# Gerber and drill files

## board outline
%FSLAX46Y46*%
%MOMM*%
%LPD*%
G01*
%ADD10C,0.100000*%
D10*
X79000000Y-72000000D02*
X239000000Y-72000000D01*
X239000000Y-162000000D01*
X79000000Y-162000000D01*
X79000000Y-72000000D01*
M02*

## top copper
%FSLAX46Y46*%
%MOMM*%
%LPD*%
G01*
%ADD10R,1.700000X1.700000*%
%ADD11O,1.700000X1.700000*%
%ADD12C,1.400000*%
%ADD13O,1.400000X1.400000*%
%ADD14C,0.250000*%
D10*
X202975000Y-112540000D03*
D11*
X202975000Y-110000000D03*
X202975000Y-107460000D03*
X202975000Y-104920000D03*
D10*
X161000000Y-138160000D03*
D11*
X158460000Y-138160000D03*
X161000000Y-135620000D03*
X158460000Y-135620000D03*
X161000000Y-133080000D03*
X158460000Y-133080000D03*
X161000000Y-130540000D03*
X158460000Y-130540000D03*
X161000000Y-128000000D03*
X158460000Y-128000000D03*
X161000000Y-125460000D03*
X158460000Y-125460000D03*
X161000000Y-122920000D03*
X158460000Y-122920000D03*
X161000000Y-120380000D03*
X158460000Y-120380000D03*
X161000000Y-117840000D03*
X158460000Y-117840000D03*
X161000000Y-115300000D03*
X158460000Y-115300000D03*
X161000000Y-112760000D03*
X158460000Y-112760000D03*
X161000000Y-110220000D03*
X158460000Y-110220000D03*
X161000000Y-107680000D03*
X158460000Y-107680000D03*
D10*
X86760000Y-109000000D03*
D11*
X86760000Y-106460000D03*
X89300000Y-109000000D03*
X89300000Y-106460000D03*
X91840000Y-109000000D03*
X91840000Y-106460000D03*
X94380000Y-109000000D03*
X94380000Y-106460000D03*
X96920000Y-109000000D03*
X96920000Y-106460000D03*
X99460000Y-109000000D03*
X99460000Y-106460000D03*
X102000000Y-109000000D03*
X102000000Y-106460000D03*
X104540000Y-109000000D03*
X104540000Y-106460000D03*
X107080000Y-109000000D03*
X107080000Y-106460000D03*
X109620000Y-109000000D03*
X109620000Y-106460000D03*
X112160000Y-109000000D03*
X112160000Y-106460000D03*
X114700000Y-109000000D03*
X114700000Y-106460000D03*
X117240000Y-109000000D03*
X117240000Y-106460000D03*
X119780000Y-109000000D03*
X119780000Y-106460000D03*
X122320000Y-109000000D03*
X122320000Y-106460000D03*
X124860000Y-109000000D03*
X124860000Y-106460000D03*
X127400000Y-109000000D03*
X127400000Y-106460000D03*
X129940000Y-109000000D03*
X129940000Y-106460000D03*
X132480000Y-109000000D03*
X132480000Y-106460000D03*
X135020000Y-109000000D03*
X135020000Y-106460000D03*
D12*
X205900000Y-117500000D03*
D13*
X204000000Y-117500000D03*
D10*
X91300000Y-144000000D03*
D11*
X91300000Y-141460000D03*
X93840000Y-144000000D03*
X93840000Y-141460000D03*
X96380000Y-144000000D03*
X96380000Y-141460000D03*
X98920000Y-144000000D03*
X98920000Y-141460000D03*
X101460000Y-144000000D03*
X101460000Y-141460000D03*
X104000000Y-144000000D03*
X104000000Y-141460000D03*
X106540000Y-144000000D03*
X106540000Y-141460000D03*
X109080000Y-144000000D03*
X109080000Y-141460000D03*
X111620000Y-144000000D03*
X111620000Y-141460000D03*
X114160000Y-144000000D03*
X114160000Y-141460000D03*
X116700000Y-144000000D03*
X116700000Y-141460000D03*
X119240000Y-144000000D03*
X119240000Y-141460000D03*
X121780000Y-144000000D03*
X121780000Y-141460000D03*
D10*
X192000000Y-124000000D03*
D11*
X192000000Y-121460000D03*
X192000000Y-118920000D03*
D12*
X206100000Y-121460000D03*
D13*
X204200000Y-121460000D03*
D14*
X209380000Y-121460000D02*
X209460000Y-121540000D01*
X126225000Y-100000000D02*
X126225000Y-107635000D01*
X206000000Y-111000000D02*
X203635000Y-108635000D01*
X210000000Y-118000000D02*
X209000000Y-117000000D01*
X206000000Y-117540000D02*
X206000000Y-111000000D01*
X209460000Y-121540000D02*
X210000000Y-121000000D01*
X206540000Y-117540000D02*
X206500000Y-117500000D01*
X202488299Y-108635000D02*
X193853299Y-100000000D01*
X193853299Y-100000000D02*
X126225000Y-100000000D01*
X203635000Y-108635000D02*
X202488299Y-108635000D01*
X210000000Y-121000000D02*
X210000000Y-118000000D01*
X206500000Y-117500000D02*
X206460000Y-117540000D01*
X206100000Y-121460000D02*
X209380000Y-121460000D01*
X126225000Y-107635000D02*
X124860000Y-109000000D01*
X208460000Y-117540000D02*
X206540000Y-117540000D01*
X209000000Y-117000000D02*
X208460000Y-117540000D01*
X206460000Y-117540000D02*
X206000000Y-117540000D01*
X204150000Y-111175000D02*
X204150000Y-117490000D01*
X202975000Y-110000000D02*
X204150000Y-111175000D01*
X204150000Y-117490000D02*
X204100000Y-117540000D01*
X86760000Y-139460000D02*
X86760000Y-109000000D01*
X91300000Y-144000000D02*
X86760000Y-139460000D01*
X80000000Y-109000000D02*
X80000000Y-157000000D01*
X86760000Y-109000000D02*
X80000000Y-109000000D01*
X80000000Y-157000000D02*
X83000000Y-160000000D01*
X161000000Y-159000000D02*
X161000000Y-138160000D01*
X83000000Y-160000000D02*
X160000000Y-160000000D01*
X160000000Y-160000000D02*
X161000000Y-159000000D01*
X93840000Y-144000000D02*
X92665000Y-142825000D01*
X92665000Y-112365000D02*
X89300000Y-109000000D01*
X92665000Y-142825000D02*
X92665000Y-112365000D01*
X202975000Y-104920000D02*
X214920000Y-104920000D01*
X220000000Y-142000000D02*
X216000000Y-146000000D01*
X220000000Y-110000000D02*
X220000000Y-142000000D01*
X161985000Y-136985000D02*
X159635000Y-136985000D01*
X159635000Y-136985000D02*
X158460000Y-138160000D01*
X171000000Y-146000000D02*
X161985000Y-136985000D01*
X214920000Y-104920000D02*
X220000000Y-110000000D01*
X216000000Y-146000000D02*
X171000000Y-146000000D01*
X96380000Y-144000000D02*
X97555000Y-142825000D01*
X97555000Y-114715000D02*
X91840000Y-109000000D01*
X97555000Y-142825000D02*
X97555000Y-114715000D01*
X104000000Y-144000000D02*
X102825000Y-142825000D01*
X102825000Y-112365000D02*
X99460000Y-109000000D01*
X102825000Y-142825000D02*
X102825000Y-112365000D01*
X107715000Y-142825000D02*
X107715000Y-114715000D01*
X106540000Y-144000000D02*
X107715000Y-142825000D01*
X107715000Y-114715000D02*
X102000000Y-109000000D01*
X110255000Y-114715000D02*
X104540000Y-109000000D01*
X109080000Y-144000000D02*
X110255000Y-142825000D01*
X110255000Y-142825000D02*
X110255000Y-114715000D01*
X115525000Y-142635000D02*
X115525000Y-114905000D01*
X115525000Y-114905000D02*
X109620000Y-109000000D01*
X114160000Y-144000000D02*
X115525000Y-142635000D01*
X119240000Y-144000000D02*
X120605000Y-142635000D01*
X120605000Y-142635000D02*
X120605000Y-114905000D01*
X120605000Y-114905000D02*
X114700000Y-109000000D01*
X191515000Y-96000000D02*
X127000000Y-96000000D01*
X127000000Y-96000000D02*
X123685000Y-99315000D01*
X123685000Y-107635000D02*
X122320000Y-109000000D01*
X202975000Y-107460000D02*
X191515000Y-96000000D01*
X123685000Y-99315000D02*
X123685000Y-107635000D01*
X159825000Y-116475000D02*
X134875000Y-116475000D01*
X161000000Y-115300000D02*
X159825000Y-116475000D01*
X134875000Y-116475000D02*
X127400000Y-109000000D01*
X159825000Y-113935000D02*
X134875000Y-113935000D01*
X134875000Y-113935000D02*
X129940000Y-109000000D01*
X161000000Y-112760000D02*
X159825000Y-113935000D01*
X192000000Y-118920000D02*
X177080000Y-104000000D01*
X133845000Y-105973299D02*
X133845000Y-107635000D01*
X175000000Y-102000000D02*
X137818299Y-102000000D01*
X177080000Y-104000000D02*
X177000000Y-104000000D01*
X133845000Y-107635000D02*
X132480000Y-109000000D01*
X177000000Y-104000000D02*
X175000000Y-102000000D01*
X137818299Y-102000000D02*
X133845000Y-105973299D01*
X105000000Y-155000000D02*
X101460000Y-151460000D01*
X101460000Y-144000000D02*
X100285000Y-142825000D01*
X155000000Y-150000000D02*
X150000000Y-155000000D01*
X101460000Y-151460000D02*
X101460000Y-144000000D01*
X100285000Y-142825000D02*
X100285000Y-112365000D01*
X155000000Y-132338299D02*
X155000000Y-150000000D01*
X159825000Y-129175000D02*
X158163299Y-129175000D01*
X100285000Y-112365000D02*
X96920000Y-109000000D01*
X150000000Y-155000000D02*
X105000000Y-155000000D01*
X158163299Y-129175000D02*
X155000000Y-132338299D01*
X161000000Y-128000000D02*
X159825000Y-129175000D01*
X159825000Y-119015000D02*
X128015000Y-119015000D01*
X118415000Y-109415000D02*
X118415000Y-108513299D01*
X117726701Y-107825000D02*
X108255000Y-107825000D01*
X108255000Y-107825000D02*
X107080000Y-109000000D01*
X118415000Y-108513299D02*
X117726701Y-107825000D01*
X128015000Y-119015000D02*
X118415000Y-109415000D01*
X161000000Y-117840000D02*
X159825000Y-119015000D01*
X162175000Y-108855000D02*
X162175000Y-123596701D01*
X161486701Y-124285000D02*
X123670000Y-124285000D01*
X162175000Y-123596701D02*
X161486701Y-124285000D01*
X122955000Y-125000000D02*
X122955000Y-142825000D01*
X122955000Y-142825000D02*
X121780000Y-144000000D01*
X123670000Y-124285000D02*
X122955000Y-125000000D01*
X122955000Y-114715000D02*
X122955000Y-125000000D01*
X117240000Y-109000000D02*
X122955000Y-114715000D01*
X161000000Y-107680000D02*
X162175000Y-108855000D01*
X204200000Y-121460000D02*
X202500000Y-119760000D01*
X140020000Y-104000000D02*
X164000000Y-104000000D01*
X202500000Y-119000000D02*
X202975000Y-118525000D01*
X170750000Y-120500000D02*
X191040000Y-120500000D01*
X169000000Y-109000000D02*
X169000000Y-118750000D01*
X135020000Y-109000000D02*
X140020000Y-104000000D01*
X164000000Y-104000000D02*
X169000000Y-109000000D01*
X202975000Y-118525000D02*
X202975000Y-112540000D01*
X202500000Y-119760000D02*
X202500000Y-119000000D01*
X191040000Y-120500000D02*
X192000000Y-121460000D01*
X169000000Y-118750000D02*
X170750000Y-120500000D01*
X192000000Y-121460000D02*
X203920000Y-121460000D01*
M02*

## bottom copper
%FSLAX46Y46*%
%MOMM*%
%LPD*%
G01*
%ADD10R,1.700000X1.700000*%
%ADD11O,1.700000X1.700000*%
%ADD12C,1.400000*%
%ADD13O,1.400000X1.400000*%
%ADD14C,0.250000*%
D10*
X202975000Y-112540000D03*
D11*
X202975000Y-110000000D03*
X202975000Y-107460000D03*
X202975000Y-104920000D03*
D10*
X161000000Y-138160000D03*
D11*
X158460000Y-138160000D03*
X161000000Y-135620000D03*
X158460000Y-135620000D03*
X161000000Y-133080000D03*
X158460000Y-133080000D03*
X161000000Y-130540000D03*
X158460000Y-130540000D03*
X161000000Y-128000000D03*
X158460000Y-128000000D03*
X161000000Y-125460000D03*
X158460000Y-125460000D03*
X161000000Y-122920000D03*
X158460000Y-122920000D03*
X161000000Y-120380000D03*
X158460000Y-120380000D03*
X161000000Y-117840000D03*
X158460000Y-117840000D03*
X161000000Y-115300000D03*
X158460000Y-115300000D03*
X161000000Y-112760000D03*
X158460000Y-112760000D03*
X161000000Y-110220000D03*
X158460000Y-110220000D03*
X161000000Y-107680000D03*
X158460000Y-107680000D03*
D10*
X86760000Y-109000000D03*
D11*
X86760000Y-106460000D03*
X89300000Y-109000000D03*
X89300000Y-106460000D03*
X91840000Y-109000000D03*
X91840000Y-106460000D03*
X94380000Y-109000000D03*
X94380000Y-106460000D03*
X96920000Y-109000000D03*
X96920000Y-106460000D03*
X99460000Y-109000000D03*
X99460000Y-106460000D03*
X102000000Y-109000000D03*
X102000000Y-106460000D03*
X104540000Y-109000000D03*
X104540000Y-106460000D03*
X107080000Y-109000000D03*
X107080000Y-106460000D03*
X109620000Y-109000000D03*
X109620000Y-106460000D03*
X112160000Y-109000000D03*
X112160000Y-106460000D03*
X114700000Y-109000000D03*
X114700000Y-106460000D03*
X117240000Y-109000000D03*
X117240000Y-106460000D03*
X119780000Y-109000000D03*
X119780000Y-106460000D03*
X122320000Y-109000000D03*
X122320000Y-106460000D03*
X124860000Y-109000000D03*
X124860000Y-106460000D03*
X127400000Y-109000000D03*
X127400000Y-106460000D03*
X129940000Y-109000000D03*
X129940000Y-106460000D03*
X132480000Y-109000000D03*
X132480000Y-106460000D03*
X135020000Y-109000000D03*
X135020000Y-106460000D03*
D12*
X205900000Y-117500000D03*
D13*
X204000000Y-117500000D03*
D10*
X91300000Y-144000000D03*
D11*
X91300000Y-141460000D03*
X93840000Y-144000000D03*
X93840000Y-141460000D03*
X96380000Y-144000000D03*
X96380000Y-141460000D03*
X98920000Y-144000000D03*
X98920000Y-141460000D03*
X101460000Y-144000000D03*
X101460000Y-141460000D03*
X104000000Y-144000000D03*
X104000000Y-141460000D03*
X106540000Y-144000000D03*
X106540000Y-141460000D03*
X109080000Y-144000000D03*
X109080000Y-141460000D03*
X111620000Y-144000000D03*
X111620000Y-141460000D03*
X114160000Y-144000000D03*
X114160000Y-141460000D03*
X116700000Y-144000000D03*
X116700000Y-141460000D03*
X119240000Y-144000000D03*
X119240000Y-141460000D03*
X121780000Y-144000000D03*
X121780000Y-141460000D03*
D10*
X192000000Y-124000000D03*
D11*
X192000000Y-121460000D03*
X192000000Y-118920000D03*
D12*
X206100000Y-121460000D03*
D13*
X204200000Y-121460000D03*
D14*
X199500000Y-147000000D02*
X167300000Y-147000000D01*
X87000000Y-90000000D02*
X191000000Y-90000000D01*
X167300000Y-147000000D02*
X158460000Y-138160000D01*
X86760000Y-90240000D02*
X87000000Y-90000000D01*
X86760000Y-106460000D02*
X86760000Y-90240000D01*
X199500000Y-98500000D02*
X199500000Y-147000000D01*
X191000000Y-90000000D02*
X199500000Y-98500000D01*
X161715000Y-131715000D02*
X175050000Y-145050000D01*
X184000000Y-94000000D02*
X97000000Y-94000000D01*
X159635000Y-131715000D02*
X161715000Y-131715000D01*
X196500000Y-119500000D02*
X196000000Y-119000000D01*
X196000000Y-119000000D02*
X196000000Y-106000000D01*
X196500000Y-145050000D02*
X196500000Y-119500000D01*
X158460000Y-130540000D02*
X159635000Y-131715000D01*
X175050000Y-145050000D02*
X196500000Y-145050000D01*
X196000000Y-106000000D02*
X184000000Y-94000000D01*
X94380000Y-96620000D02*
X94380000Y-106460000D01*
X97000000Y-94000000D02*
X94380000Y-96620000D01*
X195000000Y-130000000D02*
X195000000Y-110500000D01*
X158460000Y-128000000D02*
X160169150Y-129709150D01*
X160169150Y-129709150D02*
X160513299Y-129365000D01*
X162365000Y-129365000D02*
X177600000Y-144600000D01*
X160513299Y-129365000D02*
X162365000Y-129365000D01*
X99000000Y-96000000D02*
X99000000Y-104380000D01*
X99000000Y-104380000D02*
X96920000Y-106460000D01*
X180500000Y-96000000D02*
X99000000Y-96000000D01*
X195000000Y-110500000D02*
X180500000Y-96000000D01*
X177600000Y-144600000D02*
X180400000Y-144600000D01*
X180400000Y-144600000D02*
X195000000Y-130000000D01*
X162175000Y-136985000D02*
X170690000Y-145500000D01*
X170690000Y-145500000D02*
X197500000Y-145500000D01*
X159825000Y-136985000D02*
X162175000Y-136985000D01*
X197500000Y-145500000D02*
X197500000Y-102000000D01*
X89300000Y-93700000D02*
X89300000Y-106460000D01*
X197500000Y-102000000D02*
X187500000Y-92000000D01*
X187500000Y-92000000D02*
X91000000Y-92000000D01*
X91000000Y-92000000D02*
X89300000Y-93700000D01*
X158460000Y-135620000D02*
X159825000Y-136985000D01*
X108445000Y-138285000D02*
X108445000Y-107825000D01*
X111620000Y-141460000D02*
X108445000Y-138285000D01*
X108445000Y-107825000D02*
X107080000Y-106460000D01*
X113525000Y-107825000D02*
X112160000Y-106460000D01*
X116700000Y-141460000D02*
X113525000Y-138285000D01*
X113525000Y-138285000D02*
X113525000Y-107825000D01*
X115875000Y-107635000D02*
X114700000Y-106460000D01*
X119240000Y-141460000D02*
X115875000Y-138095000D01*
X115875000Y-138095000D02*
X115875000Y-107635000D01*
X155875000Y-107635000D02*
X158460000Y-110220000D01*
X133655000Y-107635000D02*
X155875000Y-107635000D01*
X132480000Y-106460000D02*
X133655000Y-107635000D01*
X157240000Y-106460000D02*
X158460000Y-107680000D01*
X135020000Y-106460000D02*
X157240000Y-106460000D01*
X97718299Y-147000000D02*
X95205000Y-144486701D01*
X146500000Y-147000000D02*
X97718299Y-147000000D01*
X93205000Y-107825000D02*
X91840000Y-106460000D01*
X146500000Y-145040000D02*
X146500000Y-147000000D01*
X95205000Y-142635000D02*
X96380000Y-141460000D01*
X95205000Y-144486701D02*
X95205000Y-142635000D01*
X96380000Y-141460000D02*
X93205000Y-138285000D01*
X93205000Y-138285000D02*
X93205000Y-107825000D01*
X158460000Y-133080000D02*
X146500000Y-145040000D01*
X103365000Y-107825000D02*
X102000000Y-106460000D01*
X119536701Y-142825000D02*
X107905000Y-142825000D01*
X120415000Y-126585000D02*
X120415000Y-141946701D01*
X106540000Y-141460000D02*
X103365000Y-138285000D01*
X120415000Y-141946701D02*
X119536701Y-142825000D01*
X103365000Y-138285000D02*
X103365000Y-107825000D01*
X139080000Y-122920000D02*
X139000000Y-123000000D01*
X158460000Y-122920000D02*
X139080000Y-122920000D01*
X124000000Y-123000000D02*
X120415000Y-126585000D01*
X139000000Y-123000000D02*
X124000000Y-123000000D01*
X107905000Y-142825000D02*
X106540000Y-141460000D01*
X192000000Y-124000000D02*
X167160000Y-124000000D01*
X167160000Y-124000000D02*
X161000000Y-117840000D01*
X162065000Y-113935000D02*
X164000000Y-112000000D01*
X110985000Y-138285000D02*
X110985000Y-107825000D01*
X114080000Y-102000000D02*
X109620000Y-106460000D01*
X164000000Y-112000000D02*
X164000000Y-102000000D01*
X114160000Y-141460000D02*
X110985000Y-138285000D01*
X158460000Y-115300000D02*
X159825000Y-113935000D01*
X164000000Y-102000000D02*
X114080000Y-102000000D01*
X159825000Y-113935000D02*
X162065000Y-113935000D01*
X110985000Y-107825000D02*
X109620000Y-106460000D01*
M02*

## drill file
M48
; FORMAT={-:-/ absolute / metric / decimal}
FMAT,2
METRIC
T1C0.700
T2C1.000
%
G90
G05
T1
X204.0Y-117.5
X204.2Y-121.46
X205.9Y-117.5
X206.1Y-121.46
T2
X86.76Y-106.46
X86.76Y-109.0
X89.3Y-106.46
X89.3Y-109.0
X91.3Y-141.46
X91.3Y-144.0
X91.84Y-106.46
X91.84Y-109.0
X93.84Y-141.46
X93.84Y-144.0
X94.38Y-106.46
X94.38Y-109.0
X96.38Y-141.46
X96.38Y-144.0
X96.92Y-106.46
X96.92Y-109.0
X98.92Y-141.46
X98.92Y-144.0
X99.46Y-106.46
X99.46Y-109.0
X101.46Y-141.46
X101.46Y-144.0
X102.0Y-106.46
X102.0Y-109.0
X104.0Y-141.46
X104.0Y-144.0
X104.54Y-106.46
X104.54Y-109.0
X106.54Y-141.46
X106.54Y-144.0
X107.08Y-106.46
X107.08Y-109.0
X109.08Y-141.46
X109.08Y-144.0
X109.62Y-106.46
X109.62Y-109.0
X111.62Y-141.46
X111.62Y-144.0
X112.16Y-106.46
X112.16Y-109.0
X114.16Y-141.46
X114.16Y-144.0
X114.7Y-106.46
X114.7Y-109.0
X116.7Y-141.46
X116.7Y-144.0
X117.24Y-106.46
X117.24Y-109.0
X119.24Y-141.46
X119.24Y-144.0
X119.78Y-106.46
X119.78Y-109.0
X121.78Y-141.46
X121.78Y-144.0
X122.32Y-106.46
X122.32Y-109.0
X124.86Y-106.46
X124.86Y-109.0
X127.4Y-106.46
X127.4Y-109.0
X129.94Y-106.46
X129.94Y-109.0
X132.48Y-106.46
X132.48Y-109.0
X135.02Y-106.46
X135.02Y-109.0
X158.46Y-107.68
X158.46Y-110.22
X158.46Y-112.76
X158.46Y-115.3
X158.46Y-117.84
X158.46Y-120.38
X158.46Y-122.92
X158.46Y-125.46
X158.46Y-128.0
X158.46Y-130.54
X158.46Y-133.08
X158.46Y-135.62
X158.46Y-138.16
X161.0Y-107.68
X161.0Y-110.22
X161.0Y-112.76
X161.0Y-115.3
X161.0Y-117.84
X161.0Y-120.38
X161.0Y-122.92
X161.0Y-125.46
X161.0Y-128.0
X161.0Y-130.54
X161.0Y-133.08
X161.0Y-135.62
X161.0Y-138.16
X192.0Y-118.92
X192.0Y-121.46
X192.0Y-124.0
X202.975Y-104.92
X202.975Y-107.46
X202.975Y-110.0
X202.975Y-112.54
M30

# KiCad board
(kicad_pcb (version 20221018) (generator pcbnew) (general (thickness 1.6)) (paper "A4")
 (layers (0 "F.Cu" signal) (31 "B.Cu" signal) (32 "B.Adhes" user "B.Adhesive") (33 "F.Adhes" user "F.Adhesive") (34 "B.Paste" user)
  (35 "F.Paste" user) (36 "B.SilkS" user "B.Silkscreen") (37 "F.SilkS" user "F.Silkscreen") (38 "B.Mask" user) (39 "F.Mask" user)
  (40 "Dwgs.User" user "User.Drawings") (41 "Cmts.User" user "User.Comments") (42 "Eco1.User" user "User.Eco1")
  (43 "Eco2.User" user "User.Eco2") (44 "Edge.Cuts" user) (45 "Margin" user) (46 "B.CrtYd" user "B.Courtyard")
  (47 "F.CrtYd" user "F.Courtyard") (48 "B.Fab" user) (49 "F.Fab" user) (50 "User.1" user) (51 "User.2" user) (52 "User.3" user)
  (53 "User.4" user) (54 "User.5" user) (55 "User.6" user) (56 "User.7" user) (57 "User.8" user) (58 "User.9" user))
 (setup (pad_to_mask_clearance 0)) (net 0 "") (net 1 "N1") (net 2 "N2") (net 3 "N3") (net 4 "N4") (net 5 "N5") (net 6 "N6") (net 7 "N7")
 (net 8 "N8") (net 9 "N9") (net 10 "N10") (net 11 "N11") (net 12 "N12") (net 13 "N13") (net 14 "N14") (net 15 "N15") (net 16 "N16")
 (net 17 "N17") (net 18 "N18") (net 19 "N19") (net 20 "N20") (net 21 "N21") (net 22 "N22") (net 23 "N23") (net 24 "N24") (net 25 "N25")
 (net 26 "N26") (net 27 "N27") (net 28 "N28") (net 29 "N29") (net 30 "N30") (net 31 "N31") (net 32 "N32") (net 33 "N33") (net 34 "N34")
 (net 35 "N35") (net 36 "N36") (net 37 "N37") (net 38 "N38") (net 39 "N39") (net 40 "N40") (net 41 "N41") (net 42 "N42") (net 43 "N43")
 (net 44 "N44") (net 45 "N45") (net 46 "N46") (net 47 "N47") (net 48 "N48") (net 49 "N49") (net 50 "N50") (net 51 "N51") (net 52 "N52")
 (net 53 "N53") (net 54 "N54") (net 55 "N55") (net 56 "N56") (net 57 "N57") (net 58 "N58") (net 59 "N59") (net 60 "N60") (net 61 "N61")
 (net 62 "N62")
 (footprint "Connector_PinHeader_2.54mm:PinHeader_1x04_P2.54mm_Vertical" (layer "F.Cu") (at 202.975 112.54 180)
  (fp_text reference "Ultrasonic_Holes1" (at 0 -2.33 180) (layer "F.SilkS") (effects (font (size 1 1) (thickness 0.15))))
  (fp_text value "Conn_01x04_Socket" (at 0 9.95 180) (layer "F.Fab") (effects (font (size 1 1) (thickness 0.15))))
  (pad "1" thru_hole rect (at 0 0 180) (size 1.7 1.7) (drill 1) (layers "*.Cu" "*.Mask") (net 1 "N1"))
  (pad "2" thru_hole oval (at 0 2.54 180) (size 1.7 1.7) (drill 1) (layers "*.Cu" "*.Mask") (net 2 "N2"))
  (pad "3" thru_hole oval (at 0 5.08 180) (size 1.7 1.7) (drill 1) (layers "*.Cu" "*.Mask") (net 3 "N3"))
  (pad "4" thru_hole oval (at 0 7.62 180) (size 1.7 1.7) (drill 1) (layers "*.Cu" "*.Mask") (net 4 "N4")))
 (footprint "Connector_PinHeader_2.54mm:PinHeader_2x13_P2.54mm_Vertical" (layer "F.Cu") (at 161 138.16 180)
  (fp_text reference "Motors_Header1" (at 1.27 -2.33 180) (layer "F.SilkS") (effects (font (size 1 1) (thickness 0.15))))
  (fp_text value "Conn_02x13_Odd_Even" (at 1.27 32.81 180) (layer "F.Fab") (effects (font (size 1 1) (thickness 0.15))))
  (pad "1" thru_hole rect (at 0 0 180) (size 1.7 1.7) (drill 1) (layers "*.Cu" "*.Mask") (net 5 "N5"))
  (pad "2" thru_hole oval (at 2.54 0 180) (size 1.7 1.7) (drill 1) (layers "*.Cu" "*.Mask") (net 4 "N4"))
  (pad "3" thru_hole oval (at 0 2.54 180) (size 1.7 1.7) (drill 1) (layers "*.Cu" "*.Mask") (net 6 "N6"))
  (pad "4" thru_hole oval (at 2.54 2.54 180) (size 1.7 1.7) (drill 1) (layers "*.Cu" "*.Mask") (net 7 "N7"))
  (pad "5" thru_hole oval (at 0 5.08 180) (size 1.7 1.7) (drill 1) (layers "*.Cu" "*.Mask") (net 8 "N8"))
  (pad "6" thru_hole oval (at 2.54 5.08 180) (size 1.7 1.7) (drill 1) (layers "*.Cu" "*.Mask") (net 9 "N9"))
  (pad "7" thru_hole oval (at 0 7.62 180) (size 1.7 1.7) (drill 1) (layers "*.Cu" "*.Mask") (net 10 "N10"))
  (pad "8" thru_hole oval (at 2.54 7.62 180) (size 1.7 1.7) (drill 1) (layers "*.Cu" "*.Mask") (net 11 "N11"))
  (pad "9" thru_hole oval (at 0 10.16 180) (size 1.7 1.7) (drill 1) (layers "*.Cu" "*.Mask") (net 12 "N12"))
  (pad "10" thru_hole oval (at 2.54 10.16 180) (size 1.7 1.7) (drill 1) (layers "*.Cu" "*.Mask") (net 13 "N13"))
  (pad "11" thru_hole oval (at 0 12.7 180) (size 1.7 1.7) (drill 1) (layers "*.Cu" "*.Mask") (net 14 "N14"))
  (pad "12" thru_hole oval (at 2.54 12.7 180) (size 1.7 1.7) (drill 1) (layers "*.Cu" "*.Mask") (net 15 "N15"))
  (pad "13" thru_hole oval (at 0 15.24 180) (size 1.7 1.7) (drill 1) (layers "*.Cu" "*.Mask") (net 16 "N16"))
  (pad "14" thru_hole oval (at 2.54 15.24 180) (size 1.7 1.7) (drill 1) (layers "*.Cu" "*.Mask") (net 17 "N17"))
  (pad "15" thru_hole oval (at 0 17.78 180) (size 1.7 1.7) (drill 1) (layers "*.Cu" "*.Mask") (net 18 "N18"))
  (pad "16" thru_hole oval (at 2.54 17.78 180) (size 1.7 1.7) (drill 1) (layers "*.Cu" "*.Mask") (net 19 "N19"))
  (pad "17" thru_hole oval (at 0 20.32 180) (size 1.7 1.7) (drill 1) (layers "*.Cu" "*.Mask") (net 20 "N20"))
  (pad "18" thru_hole oval (at 2.54 20.32 180) (size 1.7 1.7) (drill 1) (layers "*.Cu" "*.Mask") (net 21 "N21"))
  (pad "19" thru_hole oval (at 0 22.86 180) (size 1.7 1.7) (drill 1) (layers "*.Cu" "*.Mask") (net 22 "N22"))
  (pad "20" thru_hole oval (at 2.54 22.86 180) (size 1.7 1.7) (drill 1) (layers "*.Cu" "*.Mask") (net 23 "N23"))
  (pad "21" thru_hole oval (at 0 25.4 180) (size 1.7 1.7) (drill 1) (layers "*.Cu" "*.Mask") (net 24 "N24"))
  (pad "22" thru_hole oval (at 2.54 25.4 180) (size 1.7 1.7) (drill 1) (layers "*.Cu" "*.Mask") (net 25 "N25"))
  (pad "23" thru_hole oval (at 0 27.94 180) (size 1.7 1.7) (drill 1) (layers "*.Cu" "*.Mask") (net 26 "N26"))
  (pad "24" thru_hole oval (at 2.54 27.94 180) (size 1.7 1.7) (drill 1) (layers "*.Cu" "*.Mask") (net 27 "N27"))
  (pad "25" thru_hole oval (at 0 30.48 180) (size 1.7 1.7) (drill 1) (layers "*.Cu" "*.Mask") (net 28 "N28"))
  (pad "26" thru_hole oval (at 2.54 30.48 180) (size 1.7 1.7) (drill 1) (layers "*.Cu" "*.Mask") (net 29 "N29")))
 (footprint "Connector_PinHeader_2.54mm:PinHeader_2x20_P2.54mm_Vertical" (layer "F.Cu") (at 86.76 109 90)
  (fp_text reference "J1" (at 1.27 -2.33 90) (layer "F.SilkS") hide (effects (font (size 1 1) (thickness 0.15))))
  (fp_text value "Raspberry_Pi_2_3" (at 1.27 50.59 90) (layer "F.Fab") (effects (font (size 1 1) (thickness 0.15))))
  (pad "1" thru_hole rect (at 0 0 90) (size 1.7 1.7) (drill 1) (layers "*.Cu" "*.Mask") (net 5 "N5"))
  (pad "2" thru_hole oval (at 2.54 0 90) (size 1.7 1.7) (drill 1) (layers "*.Cu" "*.Mask") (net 4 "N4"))
  (pad "3" thru_hole oval (at 0 2.54 90) (size 1.7 1.7) (drill 1) (layers "*.Cu" "*.Mask") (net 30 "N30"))
  (pad "4" thru_hole oval (at 2.54 2.54 90) (size 1.7 1.7) (drill 1) (layers "*.Cu" "*.Mask") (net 7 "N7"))
  (pad "5" thru_hole oval (at 0 5.08 90) (size 1.7 1.7) (drill 1) (layers "*.Cu" "*.Mask") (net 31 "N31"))
  (pad "6" thru_hole oval (at 2.54 5.08 90) (size 1.7 1.7) (drill 1) (layers "*.Cu" "*.Mask") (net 9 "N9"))
  (pad "7" thru_hole oval (at 0 7.62 90) (size 1.7 1.7) (drill 1) (layers "*.Cu" "*.Mask") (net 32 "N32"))
  (pad "8" thru_hole oval (at 2.54 7.62 90) (size 1.7 1.7) (drill 1) (layers "*.Cu" "*.Mask") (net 11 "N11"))
  (pad "9" thru_hole oval (at 0 10.16 90) (size 1.7 1.7) (drill 1) (layers "*.Cu" "*.Mask") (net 12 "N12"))
  (pad "10" thru_hole oval (at 2.54 10.16 90) (size 1.7 1.7) (drill 1) (layers "*.Cu" "*.Mask") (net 13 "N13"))
  (pad "11" thru_hole oval (at 0 12.7 90) (size 1.7 1.7) (drill 1) (layers "*.Cu" "*.Mask") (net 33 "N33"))
  (pad "12" thru_hole oval (at 2.54 12.7 90) (size 1.7 1.7) (drill 1) (layers "*.Cu" "*.Mask") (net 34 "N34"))
  (pad "13" thru_hole oval (at 0 15.24 90) (size 1.7 1.7) (drill 1) (layers "*.Cu" "*.Mask") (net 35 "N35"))
  (pad "14" thru_hole oval (at 2.54 15.24 90) (size 1.7 1.7) (drill 1) (layers "*.Cu" "*.Mask") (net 17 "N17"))
  (pad "15" thru_hole oval (at 0 17.78 90) (size 1.7 1.7) (drill 1) (layers "*.Cu" "*.Mask") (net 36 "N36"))
  (pad "16" thru_hole oval (at 2.54 17.78 90) (size 1.7 1.7) (drill 1) (layers "*.Cu" "*.Mask") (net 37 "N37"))
  (pad "17" thru_hole oval (at 0 20.32 90) (size 1.7 1.7) (drill 1) (layers "*.Cu" "*.Mask") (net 20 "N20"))
  (pad "18" thru_hole oval (at 2.54 20.32 90) (size 1.7 1.7) (drill 1) (layers "*.Cu" "*.Mask") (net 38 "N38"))
  (pad "19" thru_hole oval (at 0 22.86 90) (size 1.7 1.7) (drill 1) (layers "*.Cu" "*.Mask") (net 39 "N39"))
  (pad "20" thru_hole oval (at 2.54 22.86 90) (size 1.7 1.7) (drill 1) (layers "*.Cu" "*.Mask") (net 23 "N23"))
  (pad "21" thru_hole oval (at 0 25.4 90) (size 1.7 1.7) (drill 1) (layers "*.Cu" "*.Mask") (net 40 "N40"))
  (pad "22" thru_hole oval (at 2.54 25.4 90) (size 1.7 1.7) (drill 1) (layers "*.Cu" "*.Mask") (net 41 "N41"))
  (pad "23" thru_hole oval (at 0 27.94 90) (size 1.7 1.7) (drill 1) (layers "*.Cu" "*.Mask") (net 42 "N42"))
  (pad "24" thru_hole oval (at 2.54 27.94 90) (size 1.7 1.7) (drill 1) (layers "*.Cu" "*.Mask") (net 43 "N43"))
  (pad "25" thru_hole oval (at 0 30.48 90) (size 1.7 1.7) (drill 1) (layers "*.Cu" "*.Mask") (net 28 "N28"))
  (pad "26" thru_hole oval (at 2.54 30.48 90) (size 1.7 1.7) (drill 1) (layers "*.Cu" "*.Mask") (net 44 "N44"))
  (pad "27" thru_hole oval (at 0 33.02 90) (size 1.7 1.7) (drill 1) (layers "*.Cu" "*.Mask") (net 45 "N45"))
  (pad "28" thru_hole oval (at 2.54 33.02 90) (size 1.7 1.7) (drill 1) (layers "*.Cu" "*.Mask") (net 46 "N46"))
  (pad "29" thru_hole oval (at 0 35.56 90) (size 1.7 1.7) (drill 1) (layers "*.Cu" "*.Mask") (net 3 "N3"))
  (pad "30" thru_hole oval (at 2.54 35.56 90) (size 1.7 1.7) (drill 1) (layers "*.Cu" "*.Mask") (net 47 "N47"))
  (pad "31" thru_hole oval (at 0 38.1 90) (size 1.7 1.7) (drill 1) (layers "*.Cu" "*.Mask") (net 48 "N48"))
  (pad "32" thru_hole oval (at 2.54 38.1 90) (size 1.7 1.7) (drill 1) (layers "*.Cu" "*.Mask") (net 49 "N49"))
  (pad "33" thru_hole oval (at 0 40.64 90) (size 1.7 1.7) (drill 1) (layers "*.Cu" "*.Mask") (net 22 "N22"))
  (pad "34" thru_hole oval (at 2.54 40.64 90) (size 1.7 1.7) (drill 1) (layers "*.Cu" "*.Mask") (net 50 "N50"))
  (pad "35" thru_hole oval (at 0 43.18 90) (size 1.7 1.7) (drill 1) (layers "*.Cu" "*.Mask") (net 24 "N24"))
  (pad "36" thru_hole oval (at 2.54 43.18 90) (size 1.7 1.7) (drill 1) (layers "*.Cu" "*.Mask") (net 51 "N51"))
  (pad "37" thru_hole oval (at 0 45.72 90) (size 1.7 1.7) (drill 1) (layers "*.Cu" "*.Mask") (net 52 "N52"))
  (pad "38" thru_hole oval (at 2.54 45.72 90) (size 1.7 1.7) (drill 1) (layers "*.Cu" "*.Mask") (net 27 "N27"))
  (pad "39" thru_hole oval (at 0 48.26 90) (size 1.7 1.7) (drill 1) (layers "*.Cu" "*.Mask") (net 1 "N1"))
  (pad "40" thru_hole oval (at 2.54 48.26 90) (size 1.7 1.7) (drill 1) (layers "*.Cu" "*.Mask") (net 29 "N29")))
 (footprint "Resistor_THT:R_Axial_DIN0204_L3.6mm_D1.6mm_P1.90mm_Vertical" (layer "F.Cu") (at 205.9 117.5 180)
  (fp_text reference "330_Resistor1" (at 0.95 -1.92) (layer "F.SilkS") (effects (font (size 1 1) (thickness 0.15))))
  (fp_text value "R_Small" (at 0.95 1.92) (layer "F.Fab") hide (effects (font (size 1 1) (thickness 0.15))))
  (pad "1" thru_hole circle (at 0 0 180) (size 1.4 1.4) (drill 0.7) (layers "*.Cu" "*.Mask") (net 48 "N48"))
  (pad "2" thru_hole oval (at 1.9 0 180) (size 1.4 1.4) (drill 0.7) (layers "*.Cu" "*.Mask") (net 2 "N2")))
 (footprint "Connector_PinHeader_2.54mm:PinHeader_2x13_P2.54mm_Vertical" (layer "F.Cu") (at 91.3 144 90)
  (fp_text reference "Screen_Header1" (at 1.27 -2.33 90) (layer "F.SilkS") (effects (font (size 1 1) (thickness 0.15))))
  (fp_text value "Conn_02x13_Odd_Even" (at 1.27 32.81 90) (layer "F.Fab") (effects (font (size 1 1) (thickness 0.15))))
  (pad "1" thru_hole rect (at 0 0 90) (size 1.7 1.7) (drill 1) (layers "*.Cu" "*.Mask") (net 5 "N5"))
  (pad "2" thru_hole oval (at 2.54 0 90) (size 1.7 1.7) (drill 1) (layers "*.Cu" "*.Mask") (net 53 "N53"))
  (pad "3" thru_hole oval (at 0 2.54 90) (size 1.7 1.7) (drill 1) (layers "*.Cu" "*.Mask") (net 30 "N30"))
  (pad "4" thru_hole oval (at 2.54 2.54 90) (size 1.7 1.7) (drill 1) (layers "*.Cu" "*.Mask") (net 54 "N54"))
  (pad "5" thru_hole oval (at 0 5.08 90) (size 1.7 1.7) (drill 1) (layers "*.Cu" "*.Mask") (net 31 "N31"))
  (pad "6" thru_hole oval (at 2.54 5.08 90) (size 1.7 1.7) (drill 1) (layers "*.Cu" "*.Mask") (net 9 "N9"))
  (pad "7" thru_hole oval (at 0 7.62 90) (size 1.7 1.7) (drill 1) (layers "*.Cu" "*.Mask") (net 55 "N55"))
  (pad "8" thru_hole oval (at 2.54 7.62 90) (size 1.7 1.7) (drill 1) (layers "*.Cu" "*.Mask") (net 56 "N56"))
  (pad "9" thru_hole oval (at 0 10.16 90) (size 1.7 1.7) (drill 1) (layers "*.Cu" "*.Mask") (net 12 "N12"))
  (pad "10" thru_hole oval (at 2.54 10.16 90) (size 1.7 1.7) (drill 1) (layers "*.Cu" "*.Mask") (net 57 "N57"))
  (pad "11" thru_hole oval (at 0 12.7 90) (size 1.7 1.7) (drill 1) (layers "*.Cu" "*.Mask") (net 33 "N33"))
  (pad "12" thru_hole oval (at 2.54 12.7 90) (size 1.7 1.7) (drill 1) (layers "*.Cu" "*.Mask") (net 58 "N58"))
  (pad "13" thru_hole oval (at 0 15.24 90) (size 1.7 1.7) (drill 1) (layers "*.Cu" "*.Mask") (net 35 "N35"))
  (pad "14" thru_hole oval (at 2.54 15.24 90) (size 1.7 1.7) (drill 1) (layers "*.Cu" "*.Mask") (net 17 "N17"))
  (pad "15" thru_hole oval (at 0 17.78 90) (size 1.7 1.7) (drill 1) (layers "*.Cu" "*.Mask") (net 36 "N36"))
  (pad "16" thru_hole oval (at 2.54 17.78 90) (size 1.7 1.7) (drill 1) (layers "*.Cu" "*.Mask") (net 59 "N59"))
  (pad "17" thru_hole oval (at 0 20.32 90) (size 1.7 1.7) (drill 1) (layers "*.Cu" "*.Mask") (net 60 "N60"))
  (pad "18" thru_hole oval (at 2.54 20.32 90) (size 1.7 1.7) (drill 1) (layers "*.Cu" "*.Mask") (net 38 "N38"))
  (pad "19" thru_hole oval (at 0 22.86 90) (size 1.7 1.7) (drill 1) (layers "*.Cu" "*.Mask") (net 39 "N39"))
  (pad "20" thru_hole oval (at 2.54 22.86 90) (size 1.7 1.7) (drill 1) (layers "*.Cu" "*.Mask") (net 23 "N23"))
  (pad "21" thru_hole oval (at 0 25.4 90) (size 1.7 1.7) (drill 1) (layers "*.Cu" "*.Mask") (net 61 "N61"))
  (pad "22" thru_hole oval (at 2.54 25.4 90) (size 1.7 1.7) (drill 1) (layers "*.Cu" "*.Mask") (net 41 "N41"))
  (pad "23" thru_hole oval (at 0 27.94 90) (size 1.7 1.7) (drill 1) (layers "*.Cu" "*.Mask") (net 42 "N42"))
  (pad "24" thru_hole oval (at 2.54 27.94 90) (size 1.7 1.7) (drill 1) (layers "*.Cu" "*.Mask") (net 43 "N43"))
  (pad "25" thru_hole oval (at 0 30.48 90) (size 1.7 1.7) (drill 1) (layers "*.Cu" "*.Mask") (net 28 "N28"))
  (pad "26" thru_hole oval (at 2.54 30.48 90) (size 1.7 1.7) (drill 1) (layers "*.Cu" "*.Mask") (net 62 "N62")))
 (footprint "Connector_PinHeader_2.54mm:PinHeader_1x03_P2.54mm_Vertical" (layer "F.Cu") (at 192 124 180)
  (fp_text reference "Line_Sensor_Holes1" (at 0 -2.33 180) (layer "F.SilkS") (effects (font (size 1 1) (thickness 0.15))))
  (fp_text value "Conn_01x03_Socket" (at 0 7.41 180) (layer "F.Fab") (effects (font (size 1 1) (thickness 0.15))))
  (pad "1" thru_hole rect (at 0 0 180) (size 1.7 1.7) (drill 1) (layers "*.Cu" "*.Mask") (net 20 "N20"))
  (pad "2" thru_hole oval (at 0 2.54 180) (size 1.7 1.7) (drill 1) (layers "*.Cu" "*.Mask") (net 1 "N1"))
  (pad "3" thru_hole oval (at 0 5.08 180) (size 1.7 1.7) (drill 1) (layers "*.Cu" "*.Mask") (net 52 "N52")))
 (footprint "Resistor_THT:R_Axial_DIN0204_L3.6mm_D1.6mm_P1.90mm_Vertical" (layer "F.Cu") (at 206.1 121.46 180)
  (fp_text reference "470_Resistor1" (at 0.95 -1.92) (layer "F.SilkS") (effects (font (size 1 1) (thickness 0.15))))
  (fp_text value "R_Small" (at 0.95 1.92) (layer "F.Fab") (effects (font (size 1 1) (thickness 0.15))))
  (pad "1" thru_hole circle (at 0 0 180) (size 1.4 1.4) (drill 0.7) (layers "*.Cu" "*.Mask") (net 48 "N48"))
  (pad "2" thru_hole oval (at 1.9 0 180) (size 1.4 1.4) (drill 0.7) (layers "*.Cu" "*.Mask") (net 1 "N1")))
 (gr_rect (start 79 72) (end 239 162) (stroke (width 0.1) (type solid)) (fill none) (layer "Edge.Cuts"))
 (segment (start 209.38 121.46) (end 209.46 121.54) (width 0.25) (layer "F.Cu") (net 48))
 (segment (start 126.225 100) (end 126.225 107.635) (width 0.25) (layer "F.Cu") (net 48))
 (segment (start 206 111) (end 203.635 108.635) (width 0.25) (layer "F.Cu") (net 48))
 (segment (start 210 118) (end 209 117) (width 0.25) (layer "F.Cu") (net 48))
 (segment (start 206 117.54) (end 206 111) (width 0.25) (layer "F.Cu") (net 48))
 (segment (start 209.46 121.54) (end 210 121) (width 0.25) (layer "F.Cu") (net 48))
 (segment (start 206.54 117.54) (end 206.5 117.5) (width 0.25) (layer "F.Cu") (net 48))
 (segment (start 202.488299 108.635) (end 193.853299 100) (width 0.25) (layer "F.Cu") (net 48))
 (segment (start 193.853299 100) (end 126.225 100) (width 0.25) (layer "F.Cu") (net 48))
 (segment (start 203.635 108.635) (end 202.488299 108.635) (width 0.25) (layer "F.Cu") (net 48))
 (segment (start 210 121) (end 210 118) (width 0.25) (layer "F.Cu") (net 48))
 (segment (start 206.5 117.5) (end 206.46 117.54) (width 0.25) (layer "F.Cu") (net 48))
 (segment (start 206.1 121.46) (end 209.38 121.46) (width 0.25) (layer "F.Cu") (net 48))
 (segment (start 126.225 107.635) (end 124.86 109) (width 0.25) (layer "F.Cu") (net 48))
 (segment (start 208.46 117.54) (end 206.54 117.54) (width 0.25) (layer "F.Cu") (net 48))
 (segment (start 209 117) (end 208.46 117.54) (width 0.25) (layer "F.Cu") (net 48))
 (segment (start 206.46 117.54) (end 206 117.54) (width 0.25) (layer "F.Cu") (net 48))
 (segment (start 204.15 111.175) (end 204.15 117.49) (width 0.25) (layer "F.Cu") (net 2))
 (segment (start 202.975 110) (end 204.15 111.175) (width 0.25) (layer "F.Cu") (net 2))
 (segment (start 204.15 117.49) (end 204.1 117.54) (width 0.25) (layer "F.Cu") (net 2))
 (segment (start 86.76 139.46) (end 86.76 109) (width 0.25) (layer "F.Cu") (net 5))
 (segment (start 91.3 144) (end 86.76 139.46) (width 0.25) (layer "F.Cu") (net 5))
 (segment (start 80 109) (end 80 157) (width 0.25) (layer "F.Cu") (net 5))
 (segment (start 86.76 109) (end 80 109) (width 0.25) (layer "F.Cu") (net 5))
 (segment (start 80 157) (end 83 160) (width 0.25) (layer "F.Cu") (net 5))
 (segment (start 161 159) (end 161 138.16) (width 0.25) (layer "F.Cu") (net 5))
 (segment (start 83 160) (end 160 160) (width 0.25) (layer "F.Cu") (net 5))
 (segment (start 160 160) (end 161 159) (width 0.25) (layer "F.Cu") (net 5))
 (segment (start 93.84 144) (end 92.665 142.825) (width 0.25) (layer "F.Cu") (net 30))
 (segment (start 92.665 112.365) (end 89.3 109) (width 0.25) (layer "F.Cu") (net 30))
 (segment (start 92.665 142.825) (end 92.665 112.365) (width 0.25) (layer "F.Cu") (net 30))
 (segment (start 202.975 104.92) (end 214.92 104.92) (width 0.25) (layer "F.Cu") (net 4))
 (segment (start 220 142) (end 216 146) (width 0.25) (layer "F.Cu") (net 4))
 (segment (start 220 110) (end 220 142) (width 0.25) (layer "F.Cu") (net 4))
 (segment (start 161.985 136.985) (end 159.635 136.985) (width 0.25) (layer "F.Cu") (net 4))
 (segment (start 159.635 136.985) (end 158.46 138.16) (width 0.25) (layer "F.Cu") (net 4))
 (segment (start 171 146) (end 161.985 136.985) (width 0.25) (layer "F.Cu") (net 4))
 (segment (start 214.92 104.92) (end 220 110) (width 0.25) (layer "F.Cu") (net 4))
 (segment (start 216 146) (end 171 146) (width 0.25) (layer "F.Cu") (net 4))
 (segment (start 199.5 147) (end 167.3 147) (width 0.25) (layer "B.Cu") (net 4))
 (segment (start 87 90) (end 191 90) (width 0.25) (layer "B.Cu") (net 4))
 (segment (start 167.3 147) (end 158.46 138.16) (width 0.25) (layer "B.Cu") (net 4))
 (segment (start 86.76 90.24) (end 87 90) (width 0.25) (layer "B.Cu") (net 4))
 (segment (start 86.76 106.46) (end 86.76 90.24) (width 0.25) (layer "B.Cu") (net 4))
 (segment (start 199.5 98.5) (end 199.5 147) (width 0.25) (layer "B.Cu") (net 4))
 (segment (start 191 90) (end 199.5 98.5) (width 0.25) (layer "B.Cu") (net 4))
 (segment (start 96.38 144) (end 97.555 142.825) (width 0.25) (layer "F.Cu") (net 31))
 (segment (start 97.555 114.715) (end 91.84 109) (width 0.25) (layer "F.Cu") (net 31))
 (segment (start 97.555 142.825) (end 97.555 114.715) (width 0.25) (layer "F.Cu") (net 31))
 (segment (start 161.715 131.715) (end 175.05 145.05) (width 0.25) (layer "B.Cu") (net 11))
 (segment (start 184 94) (end 97 94) (width 0.25) (layer "B.Cu") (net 11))
 (segment (start 159.635 131.715) (end 161.715 131.715) (width 0.25) (layer "B.Cu") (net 11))
 (segment (start 196.5 119.5) (end 196 119) (width 0.25) (layer "B.Cu") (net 11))
 (segment (start 196 119) (end 196 106) (width 0.25) (layer "B.Cu") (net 11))
 (segment (start 196.5 145.05) (end 196.5 119.5) (width 0.25) (layer "B.Cu") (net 11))
 (segment (start 158.46 130.54) (end 159.635 131.715) (width 0.25) (layer "B.Cu") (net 11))
 (segment (start 175.05 145.05) (end 196.5 145.05) (width 0.25) (layer "B.Cu") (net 11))
 (segment (start 196 106) (end 184 94) (width 0.25) (layer "B.Cu") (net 11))
 (segment (start 94.38 96.62) (end 94.38 106.46) (width 0.25) (layer "B.Cu") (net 11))
 (segment (start 97 94) (end 94.38 96.62) (width 0.25) (layer "B.Cu") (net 11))
 (segment (start 195 130) (end 195 110.5) (width 0.25) (layer "B.Cu") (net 13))
 (segment (start 158.46 128) (end 160.16915 129.70915) (width 0.25) (layer "B.Cu") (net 13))
 (segment (start 160.16915 129.70915) (end 160.513299 129.365) (width 0.25) (layer "B.Cu") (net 13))
 (segment (start 162.365 129.365) (end 177.6 144.6) (width 0.25) (layer "B.Cu") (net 13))
 (segment (start 160.513299 129.365) (end 162.365 129.365) (width 0.25) (layer "B.Cu") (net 13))
 (segment (start 99 96) (end 99 104.38) (width 0.25) (layer "B.Cu") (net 13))
 (segment (start 99 104.38) (end 96.92 106.46) (width 0.25) (layer "B.Cu") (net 13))
 (segment (start 180.5 96) (end 99 96) (width 0.25) (layer "B.Cu") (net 13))
 (segment (start 195 110.5) (end 180.5 96) (width 0.25) (layer "B.Cu") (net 13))
 (segment (start 177.6 144.6) (end 180.4 144.6) (width 0.25) (layer "B.Cu") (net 13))
 (segment (start 180.4 144.6) (end 195 130) (width 0.25) (layer "B.Cu") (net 13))
 (segment (start 104 144) (end 102.825 142.825) (width 0.25) (layer "F.Cu") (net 33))
 (segment (start 102.825 112.365) (end 99.46 109) (width 0.25) (layer "F.Cu") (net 33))
 (segment (start 102.825 142.825) (end 102.825 112.365) (width 0.25) (layer "F.Cu") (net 33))
 (segment (start 107.715 142.825) (end 107.715 114.715) (width 0.25) (layer "F.Cu") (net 35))
 (segment (start 106.54 144) (end 107.715 142.825) (width 0.25) (layer "F.Cu") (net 35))
 (segment (start 107.715 114.715) (end 102 109) (width 0.25) (layer "F.Cu") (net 35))
 (segment (start 110.255 114.715) (end 104.54 109) (width 0.25) (layer "F.Cu") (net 36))
 (segment (start 109.08 144) (end 110.255 142.825) (width 0.25) (layer "F.Cu") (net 36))
 (segment (start 110.255 142.825) (end 110.255 114.715) (width 0.25) (layer "F.Cu") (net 36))
 (segment (start 162.175 136.985) (end 170.69 145.5) (width 0.25) (layer "B.Cu") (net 7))
 (segment (start 170.69 145.5) (end 197.5 145.5) (width 0.25) (layer "B.Cu") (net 7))
 (segment (start 159.825 136.985) (end 162.175 136.985) (width 0.25) (layer "B.Cu") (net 7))
 (segment (start 197.5 145.5) (end 197.5 102) (width 0.25) (layer "B.Cu") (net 7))
 (segment (start 89.3 93.7) (end 89.3 106.46) (width 0.25) (layer "B.Cu") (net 7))
 (segment (start 197.5 102) (end 187.5 92) (width 0.25) (layer "B.Cu") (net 7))
 (segment (start 187.5 92) (end 91 92) (width 0.25) (layer "B.Cu") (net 7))
 (segment (start 91 92) (end 89.3 93.7) (width 0.25) (layer "B.Cu") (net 7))
 (segment (start 158.46 135.62) (end 159.825 136.985) (width 0.25) (layer "B.Cu") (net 7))
 (segment (start 108.445 138.285) (end 108.445 107.825) (width 0.25) (layer "B.Cu") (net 38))
 (segment (start 111.62 141.46) (end 108.445 138.285) (width 0.25) (layer "B.Cu") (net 38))
 (segment (start 108.445 107.825) (end 107.08 106.46) (width 0.25) (layer "B.Cu") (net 38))
 (segment (start 115.525 142.635) (end 115.525 114.905) (width 0.25) (layer "F.Cu") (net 39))
 (segment (start 115.525 114.905) (end 109.62 109) (width 0.25) (layer "F.Cu") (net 39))
 (segment (start 114.16 144) (end 115.525 142.635) (width 0.25) (layer "F.Cu") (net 39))
 (segment (start 113.525 107.825) (end 112.16 106.46) (width 0.25) (layer "B.Cu") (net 41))
 (segment (start 116.7 141.46) (end 113.525 138.285) (width 0.25) (layer "B.Cu") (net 41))
 (segment (start 113.525 138.285) (end 113.525 107.825) (width 0.25) (layer "B.Cu") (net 41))
 (segment (start 119.24 144) (end 120.605 142.635) (width 0.25) (layer "F.Cu") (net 42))
 (segment (start 120.605 142.635) (end 120.605 114.905) (width 0.25) (layer "F.Cu") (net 42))
 (segment (start 120.605 114.905) (end 114.7 109) (width 0.25) (layer "F.Cu") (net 42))
 (segment (start 115.875 107.635) (end 114.7 106.46) (width 0.25) (layer "B.Cu") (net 43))
 (segment (start 119.24 141.46) (end 115.875 138.095) (width 0.25) (layer "B.Cu") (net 43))
 (segment (start 115.875 138.095) (end 115.875 107.635) (width 0.25) (layer "B.Cu") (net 43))
 (segment (start 191.515 96) (end 127 96) (width 0.25) (layer "F.Cu") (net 3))
 (segment (start 127 96) (end 123.685 99.315) (width 0.25) (layer "F.Cu") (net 3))
 (segment (start 123.685 107.635) (end 122.32 109) (width 0.25) (layer "F.Cu") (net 3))
 (segment (start 202.975 107.46) (end 191.515 96) (width 0.25) (layer "F.Cu") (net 3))
 (segment (start 123.685 99.315) (end 123.685 107.635) (width 0.25) (layer "F.Cu") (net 3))
 (segment (start 159.825 116.475) (end 134.875 116.475) (width 0.25) (layer "F.Cu") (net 22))
 (segment (start 161 115.3) (end 159.825 116.475) (width 0.25) (layer "F.Cu") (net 22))
 (segment (start 134.875 116.475) (end 127.4 109) (width 0.25) (layer "F.Cu") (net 22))
 (segment (start 159.825 113.935) (end 134.875 113.935) (width 0.25) (layer "F.Cu") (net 24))
 (segment (start 134.875 113.935) (end 129.94 109) (width 0.25) (layer "F.Cu") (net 24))
 (segment (start 161 112.76) (end 159.825 113.935) (width 0.25) (layer "F.Cu") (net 24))
 (segment (start 192 118.92) (end 177.08 104) (width 0.25) (layer "F.Cu") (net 52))
 (segment (start 133.845 105.973299) (end 133.845 107.635) (width 0.25) (layer "F.Cu") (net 52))
 (segment (start 175 102) (end 137.818299 102) (width 0.25) (layer "F.Cu") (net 52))
 (segment (start 177.08 104) (end 177 104) (width 0.25) (layer "F.Cu") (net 52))
 (segment (start 133.845 107.635) (end 132.48 109) (width 0.25) (layer "F.Cu") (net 52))
 (segment (start 177 104) (end 175 102) (width 0.25) (layer "F.Cu") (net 52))
 (segment (start 137.818299 102) (end 133.845 105.973299) (width 0.25) (layer "F.Cu") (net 52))
 (segment (start 155.875 107.635) (end 158.46 110.22) (width 0.25) (layer "B.Cu") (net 27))
 (segment (start 133.655 107.635) (end 155.875 107.635) (width 0.25) (layer "B.Cu") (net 27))
 (segment (start 132.48 106.46) (end 133.655 107.635) (width 0.25) (layer "B.Cu") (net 27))
 (segment (start 157.24 106.46) (end 158.46 107.68) (width 0.25) (layer "B.Cu") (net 29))
 (segment (start 135.02 106.46) (end 157.24 106.46) (width 0.25) (layer "B.Cu") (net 29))
 (segment (start 97.718299 147) (end 95.205 144.486701) (width 0.25) (layer "B.Cu") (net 9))
 (segment (start 146.5 147) (end 97.718299 147) (width 0.25) (layer "B.Cu") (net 9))
 (segment (start 93.205 107.825) (end 91.84 106.46) (width 0.25) (layer "B.Cu") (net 9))
 (segment (start 146.5 145.04) (end 146.5 147) (width 0.25) (layer "B.Cu") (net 9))
 (segment (start 95.205 142.635) (end 96.38 141.46) (width 0.25) (layer "B.Cu") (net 9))
 (segment (start 95.205 144.486701) (end 95.205 142.635) (width 0.25) (layer "B.Cu") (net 9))
 (segment (start 96.38 141.46) (end 93.205 138.285) (width 0.25) (layer "B.Cu") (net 9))
 (segment (start 93.205 138.285) (end 93.205 107.825) (width 0.25) (layer "B.Cu") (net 9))
 (segment (start 158.46 133.08) (end 146.5 145.04) (width 0.25) (layer "B.Cu") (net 9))
 (segment (start 105 155) (end 101.46 151.46) (width 0.25) (layer "F.Cu") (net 12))
 (segment (start 101.46 144) (end 100.285 142.825) (width 0.25) (layer "F.Cu") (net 12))
 (segment (start 155 150) (end 150 155) (width 0.25) (layer "F.Cu") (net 12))
 (segment (start 101.46 151.46) (end 101.46 144) (width 0.25) (layer "F.Cu") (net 12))
 (segment (start 100.285 142.825) (end 100.285 112.365) (width 0.25) (layer "F.Cu") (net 12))
 (segment (start 155 132.338299) (end 155 150) (width 0.25) (layer "F.Cu") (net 12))
 (segment (start 159.825 129.175) (end 158.163299 129.175) (width 0.25) (layer "F.Cu") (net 12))
 (segment (start 100.285 112.365) (end 96.92 109) (width 0.25) (layer "F.Cu") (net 12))
 (segment (start 150 155) (end 105 155) (width 0.25) (layer "F.Cu") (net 12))
 (segment (start 158.163299 129.175) (end 155 132.338299) (width 0.25) (layer "F.Cu") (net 12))
 (segment (start 161 128) (end 159.825 129.175) (width 0.25) (layer "F.Cu") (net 12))
 (segment (start 103.365 107.825) (end 102 106.46) (width 0.25) (layer "B.Cu") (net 17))
 (segment (start 119.536701 142.825) (end 107.905 142.825) (width 0.25) (layer "B.Cu") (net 17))
 (segment (start 120.415 126.585) (end 120.415 141.946701) (width 0.25) (layer "B.Cu") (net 17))
 (segment (start 106.54 141.46) (end 103.365 138.285) (width 0.25) (layer "B.Cu") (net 17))
 (segment (start 120.415 141.946701) (end 119.536701 142.825) (width 0.25) (layer "B.Cu") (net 17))
 (segment (start 103.365 138.285) (end 103.365 107.825) (width 0.25) (layer "B.Cu") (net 17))
 (segment (start 139.08 122.92) (end 139 123) (width 0.25) (layer "B.Cu") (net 17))
 (segment (start 158.46 122.92) (end 139.08 122.92) (width 0.25) (layer "B.Cu") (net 17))
 (segment (start 124 123) (end 120.415 126.585) (width 0.25) (layer "B.Cu") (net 17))
 (segment (start 139 123) (end 124 123) (width 0.25) (layer "B.Cu") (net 17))
 (segment (start 107.905 142.825) (end 106.54 141.46) (width 0.25) (layer "B.Cu") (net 17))
 (segment (start 159.825 119.015) (end 128.015 119.015) (width 0.25) (layer "F.Cu") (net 20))
 (segment (start 118.415 109.415) (end 118.415 108.513299) (width 0.25) (layer "F.Cu") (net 20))
 (segment (start 117.726701 107.825) (end 108.255 107.825) (width 0.25) (layer "F.Cu") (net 20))
 (segment (start 108.255 107.825) (end 107.08 109) (width 0.25) (layer "F.Cu") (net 20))
 (segment (start 118.415 108.513299) (end 117.726701 107.825) (width 0.25) (layer "F.Cu") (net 20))
 (segment (start 128.015 119.015) (end 118.415 109.415) (width 0.25) (layer "F.Cu") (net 20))
 (segment (start 161 117.84) (end 159.825 119.015) (width 0.25) (layer "F.Cu") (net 20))
 (segment (start 192 124) (end 167.16 124) (width 0.25) (layer "B.Cu") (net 20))
 (segment (start 167.16 124) (end 161 117.84) (width 0.25) (layer "B.Cu") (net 20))
 (segment (start 162.065 113.935) (end 164 112) (width 0.25) (layer "B.Cu") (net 23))
 (segment (start 110.985 138.285) (end 110.985 107.825) (width 0.25) (layer "B.Cu") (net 23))
 (segment (start 114.08 102) (end 109.62 106.46) (width 0.25) (layer "B.Cu") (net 23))
 (segment (start 164 112) (end 164 102) (width 0.25) (layer "B.Cu") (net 23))
 (segment (start 114.16 141.46) (end 110.985 138.285) (width 0.25) (layer "B.Cu") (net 23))
 (segment (start 158.46 115.3) (end 159.825 113.935) (width 0.25) (layer "B.Cu") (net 23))
 (segment (start 164 102) (end 114.08 102) (width 0.25) (layer "B.Cu") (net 23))
 (segment (start 159.825 113.935) (end 162.065 113.935) (width 0.25) (layer "B.Cu") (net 23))
 (segment (start 110.985 107.825) (end 109.62 106.46) (width 0.25) (layer "B.Cu") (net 23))
 (segment (start 162.175 108.855) (end 162.175 123.596701) (width 0.25) (layer "F.Cu") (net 28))
 (segment (start 161.486701 124.285) (end 123.67 124.285) (width 0.25) (layer "F.Cu") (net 28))
 (segment (start 162.175 123.596701) (end 161.486701 124.285) (width 0.25) (layer "F.Cu") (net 28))
 (segment (start 122.955 125) (end 122.955 142.825) (width 0.25) (layer "F.Cu") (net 28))
 (segment (start 122.955 142.825) (end 121.78 144) (width 0.25) (layer "F.Cu") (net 28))
 (segment (start 123.67 124.285) (end 122.955 125) (width 0.25) (layer "F.Cu") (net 28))
 (segment (start 122.955 114.715) (end 122.955 125) (width 0.25) (layer "F.Cu") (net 28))
 (segment (start 117.24 109) (end 122.955 114.715) (width 0.25) (layer "F.Cu") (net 28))
 (segment (start 161 107.68) (end 162.175 108.855) (width 0.25) (layer "F.Cu") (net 28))
 (segment (start 204.2 121.46) (end 202.5 119.76) (width 0.25) (layer "F.Cu") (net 1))
 (segment (start 140.02 104) (end 164 104) (width 0.25) (layer "F.Cu") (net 1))
 (segment (start 202.5 119) (end 202.975 118.525) (width 0.25) (layer "F.Cu") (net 1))
 (segment (start 170.75 120.5) (end 191.04 120.5) (width 0.25) (layer "F.Cu") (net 1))
 (segment (start 169 109) (end 169 118.75) (width 0.25) (layer "F.Cu") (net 1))
 (segment (start 135.02 109) (end 140.02 104) (width 0.25) (layer "F.Cu") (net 1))
 (segment (start 164 104) (end 169 109) (width 0.25) (layer "F.Cu") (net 1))
 (segment (start 202.975 118.525) (end 202.975 112.54) (width 0.25) (layer "F.Cu") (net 1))
 (segment (start 202.5 119.76) (end 202.5 119) (width 0.25) (layer "F.Cu") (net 1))
 (segment (start 191.04 120.5) (end 192 121.46) (width 0.25) (layer "F.Cu") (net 1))
 (segment (start 169 118.75) (end 170.75 120.5) (width 0.25) (layer "F.Cu") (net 1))
 (segment (start 192 121.46) (end 203.92 121.46) (width 0.25) (layer "F.Cu") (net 1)))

